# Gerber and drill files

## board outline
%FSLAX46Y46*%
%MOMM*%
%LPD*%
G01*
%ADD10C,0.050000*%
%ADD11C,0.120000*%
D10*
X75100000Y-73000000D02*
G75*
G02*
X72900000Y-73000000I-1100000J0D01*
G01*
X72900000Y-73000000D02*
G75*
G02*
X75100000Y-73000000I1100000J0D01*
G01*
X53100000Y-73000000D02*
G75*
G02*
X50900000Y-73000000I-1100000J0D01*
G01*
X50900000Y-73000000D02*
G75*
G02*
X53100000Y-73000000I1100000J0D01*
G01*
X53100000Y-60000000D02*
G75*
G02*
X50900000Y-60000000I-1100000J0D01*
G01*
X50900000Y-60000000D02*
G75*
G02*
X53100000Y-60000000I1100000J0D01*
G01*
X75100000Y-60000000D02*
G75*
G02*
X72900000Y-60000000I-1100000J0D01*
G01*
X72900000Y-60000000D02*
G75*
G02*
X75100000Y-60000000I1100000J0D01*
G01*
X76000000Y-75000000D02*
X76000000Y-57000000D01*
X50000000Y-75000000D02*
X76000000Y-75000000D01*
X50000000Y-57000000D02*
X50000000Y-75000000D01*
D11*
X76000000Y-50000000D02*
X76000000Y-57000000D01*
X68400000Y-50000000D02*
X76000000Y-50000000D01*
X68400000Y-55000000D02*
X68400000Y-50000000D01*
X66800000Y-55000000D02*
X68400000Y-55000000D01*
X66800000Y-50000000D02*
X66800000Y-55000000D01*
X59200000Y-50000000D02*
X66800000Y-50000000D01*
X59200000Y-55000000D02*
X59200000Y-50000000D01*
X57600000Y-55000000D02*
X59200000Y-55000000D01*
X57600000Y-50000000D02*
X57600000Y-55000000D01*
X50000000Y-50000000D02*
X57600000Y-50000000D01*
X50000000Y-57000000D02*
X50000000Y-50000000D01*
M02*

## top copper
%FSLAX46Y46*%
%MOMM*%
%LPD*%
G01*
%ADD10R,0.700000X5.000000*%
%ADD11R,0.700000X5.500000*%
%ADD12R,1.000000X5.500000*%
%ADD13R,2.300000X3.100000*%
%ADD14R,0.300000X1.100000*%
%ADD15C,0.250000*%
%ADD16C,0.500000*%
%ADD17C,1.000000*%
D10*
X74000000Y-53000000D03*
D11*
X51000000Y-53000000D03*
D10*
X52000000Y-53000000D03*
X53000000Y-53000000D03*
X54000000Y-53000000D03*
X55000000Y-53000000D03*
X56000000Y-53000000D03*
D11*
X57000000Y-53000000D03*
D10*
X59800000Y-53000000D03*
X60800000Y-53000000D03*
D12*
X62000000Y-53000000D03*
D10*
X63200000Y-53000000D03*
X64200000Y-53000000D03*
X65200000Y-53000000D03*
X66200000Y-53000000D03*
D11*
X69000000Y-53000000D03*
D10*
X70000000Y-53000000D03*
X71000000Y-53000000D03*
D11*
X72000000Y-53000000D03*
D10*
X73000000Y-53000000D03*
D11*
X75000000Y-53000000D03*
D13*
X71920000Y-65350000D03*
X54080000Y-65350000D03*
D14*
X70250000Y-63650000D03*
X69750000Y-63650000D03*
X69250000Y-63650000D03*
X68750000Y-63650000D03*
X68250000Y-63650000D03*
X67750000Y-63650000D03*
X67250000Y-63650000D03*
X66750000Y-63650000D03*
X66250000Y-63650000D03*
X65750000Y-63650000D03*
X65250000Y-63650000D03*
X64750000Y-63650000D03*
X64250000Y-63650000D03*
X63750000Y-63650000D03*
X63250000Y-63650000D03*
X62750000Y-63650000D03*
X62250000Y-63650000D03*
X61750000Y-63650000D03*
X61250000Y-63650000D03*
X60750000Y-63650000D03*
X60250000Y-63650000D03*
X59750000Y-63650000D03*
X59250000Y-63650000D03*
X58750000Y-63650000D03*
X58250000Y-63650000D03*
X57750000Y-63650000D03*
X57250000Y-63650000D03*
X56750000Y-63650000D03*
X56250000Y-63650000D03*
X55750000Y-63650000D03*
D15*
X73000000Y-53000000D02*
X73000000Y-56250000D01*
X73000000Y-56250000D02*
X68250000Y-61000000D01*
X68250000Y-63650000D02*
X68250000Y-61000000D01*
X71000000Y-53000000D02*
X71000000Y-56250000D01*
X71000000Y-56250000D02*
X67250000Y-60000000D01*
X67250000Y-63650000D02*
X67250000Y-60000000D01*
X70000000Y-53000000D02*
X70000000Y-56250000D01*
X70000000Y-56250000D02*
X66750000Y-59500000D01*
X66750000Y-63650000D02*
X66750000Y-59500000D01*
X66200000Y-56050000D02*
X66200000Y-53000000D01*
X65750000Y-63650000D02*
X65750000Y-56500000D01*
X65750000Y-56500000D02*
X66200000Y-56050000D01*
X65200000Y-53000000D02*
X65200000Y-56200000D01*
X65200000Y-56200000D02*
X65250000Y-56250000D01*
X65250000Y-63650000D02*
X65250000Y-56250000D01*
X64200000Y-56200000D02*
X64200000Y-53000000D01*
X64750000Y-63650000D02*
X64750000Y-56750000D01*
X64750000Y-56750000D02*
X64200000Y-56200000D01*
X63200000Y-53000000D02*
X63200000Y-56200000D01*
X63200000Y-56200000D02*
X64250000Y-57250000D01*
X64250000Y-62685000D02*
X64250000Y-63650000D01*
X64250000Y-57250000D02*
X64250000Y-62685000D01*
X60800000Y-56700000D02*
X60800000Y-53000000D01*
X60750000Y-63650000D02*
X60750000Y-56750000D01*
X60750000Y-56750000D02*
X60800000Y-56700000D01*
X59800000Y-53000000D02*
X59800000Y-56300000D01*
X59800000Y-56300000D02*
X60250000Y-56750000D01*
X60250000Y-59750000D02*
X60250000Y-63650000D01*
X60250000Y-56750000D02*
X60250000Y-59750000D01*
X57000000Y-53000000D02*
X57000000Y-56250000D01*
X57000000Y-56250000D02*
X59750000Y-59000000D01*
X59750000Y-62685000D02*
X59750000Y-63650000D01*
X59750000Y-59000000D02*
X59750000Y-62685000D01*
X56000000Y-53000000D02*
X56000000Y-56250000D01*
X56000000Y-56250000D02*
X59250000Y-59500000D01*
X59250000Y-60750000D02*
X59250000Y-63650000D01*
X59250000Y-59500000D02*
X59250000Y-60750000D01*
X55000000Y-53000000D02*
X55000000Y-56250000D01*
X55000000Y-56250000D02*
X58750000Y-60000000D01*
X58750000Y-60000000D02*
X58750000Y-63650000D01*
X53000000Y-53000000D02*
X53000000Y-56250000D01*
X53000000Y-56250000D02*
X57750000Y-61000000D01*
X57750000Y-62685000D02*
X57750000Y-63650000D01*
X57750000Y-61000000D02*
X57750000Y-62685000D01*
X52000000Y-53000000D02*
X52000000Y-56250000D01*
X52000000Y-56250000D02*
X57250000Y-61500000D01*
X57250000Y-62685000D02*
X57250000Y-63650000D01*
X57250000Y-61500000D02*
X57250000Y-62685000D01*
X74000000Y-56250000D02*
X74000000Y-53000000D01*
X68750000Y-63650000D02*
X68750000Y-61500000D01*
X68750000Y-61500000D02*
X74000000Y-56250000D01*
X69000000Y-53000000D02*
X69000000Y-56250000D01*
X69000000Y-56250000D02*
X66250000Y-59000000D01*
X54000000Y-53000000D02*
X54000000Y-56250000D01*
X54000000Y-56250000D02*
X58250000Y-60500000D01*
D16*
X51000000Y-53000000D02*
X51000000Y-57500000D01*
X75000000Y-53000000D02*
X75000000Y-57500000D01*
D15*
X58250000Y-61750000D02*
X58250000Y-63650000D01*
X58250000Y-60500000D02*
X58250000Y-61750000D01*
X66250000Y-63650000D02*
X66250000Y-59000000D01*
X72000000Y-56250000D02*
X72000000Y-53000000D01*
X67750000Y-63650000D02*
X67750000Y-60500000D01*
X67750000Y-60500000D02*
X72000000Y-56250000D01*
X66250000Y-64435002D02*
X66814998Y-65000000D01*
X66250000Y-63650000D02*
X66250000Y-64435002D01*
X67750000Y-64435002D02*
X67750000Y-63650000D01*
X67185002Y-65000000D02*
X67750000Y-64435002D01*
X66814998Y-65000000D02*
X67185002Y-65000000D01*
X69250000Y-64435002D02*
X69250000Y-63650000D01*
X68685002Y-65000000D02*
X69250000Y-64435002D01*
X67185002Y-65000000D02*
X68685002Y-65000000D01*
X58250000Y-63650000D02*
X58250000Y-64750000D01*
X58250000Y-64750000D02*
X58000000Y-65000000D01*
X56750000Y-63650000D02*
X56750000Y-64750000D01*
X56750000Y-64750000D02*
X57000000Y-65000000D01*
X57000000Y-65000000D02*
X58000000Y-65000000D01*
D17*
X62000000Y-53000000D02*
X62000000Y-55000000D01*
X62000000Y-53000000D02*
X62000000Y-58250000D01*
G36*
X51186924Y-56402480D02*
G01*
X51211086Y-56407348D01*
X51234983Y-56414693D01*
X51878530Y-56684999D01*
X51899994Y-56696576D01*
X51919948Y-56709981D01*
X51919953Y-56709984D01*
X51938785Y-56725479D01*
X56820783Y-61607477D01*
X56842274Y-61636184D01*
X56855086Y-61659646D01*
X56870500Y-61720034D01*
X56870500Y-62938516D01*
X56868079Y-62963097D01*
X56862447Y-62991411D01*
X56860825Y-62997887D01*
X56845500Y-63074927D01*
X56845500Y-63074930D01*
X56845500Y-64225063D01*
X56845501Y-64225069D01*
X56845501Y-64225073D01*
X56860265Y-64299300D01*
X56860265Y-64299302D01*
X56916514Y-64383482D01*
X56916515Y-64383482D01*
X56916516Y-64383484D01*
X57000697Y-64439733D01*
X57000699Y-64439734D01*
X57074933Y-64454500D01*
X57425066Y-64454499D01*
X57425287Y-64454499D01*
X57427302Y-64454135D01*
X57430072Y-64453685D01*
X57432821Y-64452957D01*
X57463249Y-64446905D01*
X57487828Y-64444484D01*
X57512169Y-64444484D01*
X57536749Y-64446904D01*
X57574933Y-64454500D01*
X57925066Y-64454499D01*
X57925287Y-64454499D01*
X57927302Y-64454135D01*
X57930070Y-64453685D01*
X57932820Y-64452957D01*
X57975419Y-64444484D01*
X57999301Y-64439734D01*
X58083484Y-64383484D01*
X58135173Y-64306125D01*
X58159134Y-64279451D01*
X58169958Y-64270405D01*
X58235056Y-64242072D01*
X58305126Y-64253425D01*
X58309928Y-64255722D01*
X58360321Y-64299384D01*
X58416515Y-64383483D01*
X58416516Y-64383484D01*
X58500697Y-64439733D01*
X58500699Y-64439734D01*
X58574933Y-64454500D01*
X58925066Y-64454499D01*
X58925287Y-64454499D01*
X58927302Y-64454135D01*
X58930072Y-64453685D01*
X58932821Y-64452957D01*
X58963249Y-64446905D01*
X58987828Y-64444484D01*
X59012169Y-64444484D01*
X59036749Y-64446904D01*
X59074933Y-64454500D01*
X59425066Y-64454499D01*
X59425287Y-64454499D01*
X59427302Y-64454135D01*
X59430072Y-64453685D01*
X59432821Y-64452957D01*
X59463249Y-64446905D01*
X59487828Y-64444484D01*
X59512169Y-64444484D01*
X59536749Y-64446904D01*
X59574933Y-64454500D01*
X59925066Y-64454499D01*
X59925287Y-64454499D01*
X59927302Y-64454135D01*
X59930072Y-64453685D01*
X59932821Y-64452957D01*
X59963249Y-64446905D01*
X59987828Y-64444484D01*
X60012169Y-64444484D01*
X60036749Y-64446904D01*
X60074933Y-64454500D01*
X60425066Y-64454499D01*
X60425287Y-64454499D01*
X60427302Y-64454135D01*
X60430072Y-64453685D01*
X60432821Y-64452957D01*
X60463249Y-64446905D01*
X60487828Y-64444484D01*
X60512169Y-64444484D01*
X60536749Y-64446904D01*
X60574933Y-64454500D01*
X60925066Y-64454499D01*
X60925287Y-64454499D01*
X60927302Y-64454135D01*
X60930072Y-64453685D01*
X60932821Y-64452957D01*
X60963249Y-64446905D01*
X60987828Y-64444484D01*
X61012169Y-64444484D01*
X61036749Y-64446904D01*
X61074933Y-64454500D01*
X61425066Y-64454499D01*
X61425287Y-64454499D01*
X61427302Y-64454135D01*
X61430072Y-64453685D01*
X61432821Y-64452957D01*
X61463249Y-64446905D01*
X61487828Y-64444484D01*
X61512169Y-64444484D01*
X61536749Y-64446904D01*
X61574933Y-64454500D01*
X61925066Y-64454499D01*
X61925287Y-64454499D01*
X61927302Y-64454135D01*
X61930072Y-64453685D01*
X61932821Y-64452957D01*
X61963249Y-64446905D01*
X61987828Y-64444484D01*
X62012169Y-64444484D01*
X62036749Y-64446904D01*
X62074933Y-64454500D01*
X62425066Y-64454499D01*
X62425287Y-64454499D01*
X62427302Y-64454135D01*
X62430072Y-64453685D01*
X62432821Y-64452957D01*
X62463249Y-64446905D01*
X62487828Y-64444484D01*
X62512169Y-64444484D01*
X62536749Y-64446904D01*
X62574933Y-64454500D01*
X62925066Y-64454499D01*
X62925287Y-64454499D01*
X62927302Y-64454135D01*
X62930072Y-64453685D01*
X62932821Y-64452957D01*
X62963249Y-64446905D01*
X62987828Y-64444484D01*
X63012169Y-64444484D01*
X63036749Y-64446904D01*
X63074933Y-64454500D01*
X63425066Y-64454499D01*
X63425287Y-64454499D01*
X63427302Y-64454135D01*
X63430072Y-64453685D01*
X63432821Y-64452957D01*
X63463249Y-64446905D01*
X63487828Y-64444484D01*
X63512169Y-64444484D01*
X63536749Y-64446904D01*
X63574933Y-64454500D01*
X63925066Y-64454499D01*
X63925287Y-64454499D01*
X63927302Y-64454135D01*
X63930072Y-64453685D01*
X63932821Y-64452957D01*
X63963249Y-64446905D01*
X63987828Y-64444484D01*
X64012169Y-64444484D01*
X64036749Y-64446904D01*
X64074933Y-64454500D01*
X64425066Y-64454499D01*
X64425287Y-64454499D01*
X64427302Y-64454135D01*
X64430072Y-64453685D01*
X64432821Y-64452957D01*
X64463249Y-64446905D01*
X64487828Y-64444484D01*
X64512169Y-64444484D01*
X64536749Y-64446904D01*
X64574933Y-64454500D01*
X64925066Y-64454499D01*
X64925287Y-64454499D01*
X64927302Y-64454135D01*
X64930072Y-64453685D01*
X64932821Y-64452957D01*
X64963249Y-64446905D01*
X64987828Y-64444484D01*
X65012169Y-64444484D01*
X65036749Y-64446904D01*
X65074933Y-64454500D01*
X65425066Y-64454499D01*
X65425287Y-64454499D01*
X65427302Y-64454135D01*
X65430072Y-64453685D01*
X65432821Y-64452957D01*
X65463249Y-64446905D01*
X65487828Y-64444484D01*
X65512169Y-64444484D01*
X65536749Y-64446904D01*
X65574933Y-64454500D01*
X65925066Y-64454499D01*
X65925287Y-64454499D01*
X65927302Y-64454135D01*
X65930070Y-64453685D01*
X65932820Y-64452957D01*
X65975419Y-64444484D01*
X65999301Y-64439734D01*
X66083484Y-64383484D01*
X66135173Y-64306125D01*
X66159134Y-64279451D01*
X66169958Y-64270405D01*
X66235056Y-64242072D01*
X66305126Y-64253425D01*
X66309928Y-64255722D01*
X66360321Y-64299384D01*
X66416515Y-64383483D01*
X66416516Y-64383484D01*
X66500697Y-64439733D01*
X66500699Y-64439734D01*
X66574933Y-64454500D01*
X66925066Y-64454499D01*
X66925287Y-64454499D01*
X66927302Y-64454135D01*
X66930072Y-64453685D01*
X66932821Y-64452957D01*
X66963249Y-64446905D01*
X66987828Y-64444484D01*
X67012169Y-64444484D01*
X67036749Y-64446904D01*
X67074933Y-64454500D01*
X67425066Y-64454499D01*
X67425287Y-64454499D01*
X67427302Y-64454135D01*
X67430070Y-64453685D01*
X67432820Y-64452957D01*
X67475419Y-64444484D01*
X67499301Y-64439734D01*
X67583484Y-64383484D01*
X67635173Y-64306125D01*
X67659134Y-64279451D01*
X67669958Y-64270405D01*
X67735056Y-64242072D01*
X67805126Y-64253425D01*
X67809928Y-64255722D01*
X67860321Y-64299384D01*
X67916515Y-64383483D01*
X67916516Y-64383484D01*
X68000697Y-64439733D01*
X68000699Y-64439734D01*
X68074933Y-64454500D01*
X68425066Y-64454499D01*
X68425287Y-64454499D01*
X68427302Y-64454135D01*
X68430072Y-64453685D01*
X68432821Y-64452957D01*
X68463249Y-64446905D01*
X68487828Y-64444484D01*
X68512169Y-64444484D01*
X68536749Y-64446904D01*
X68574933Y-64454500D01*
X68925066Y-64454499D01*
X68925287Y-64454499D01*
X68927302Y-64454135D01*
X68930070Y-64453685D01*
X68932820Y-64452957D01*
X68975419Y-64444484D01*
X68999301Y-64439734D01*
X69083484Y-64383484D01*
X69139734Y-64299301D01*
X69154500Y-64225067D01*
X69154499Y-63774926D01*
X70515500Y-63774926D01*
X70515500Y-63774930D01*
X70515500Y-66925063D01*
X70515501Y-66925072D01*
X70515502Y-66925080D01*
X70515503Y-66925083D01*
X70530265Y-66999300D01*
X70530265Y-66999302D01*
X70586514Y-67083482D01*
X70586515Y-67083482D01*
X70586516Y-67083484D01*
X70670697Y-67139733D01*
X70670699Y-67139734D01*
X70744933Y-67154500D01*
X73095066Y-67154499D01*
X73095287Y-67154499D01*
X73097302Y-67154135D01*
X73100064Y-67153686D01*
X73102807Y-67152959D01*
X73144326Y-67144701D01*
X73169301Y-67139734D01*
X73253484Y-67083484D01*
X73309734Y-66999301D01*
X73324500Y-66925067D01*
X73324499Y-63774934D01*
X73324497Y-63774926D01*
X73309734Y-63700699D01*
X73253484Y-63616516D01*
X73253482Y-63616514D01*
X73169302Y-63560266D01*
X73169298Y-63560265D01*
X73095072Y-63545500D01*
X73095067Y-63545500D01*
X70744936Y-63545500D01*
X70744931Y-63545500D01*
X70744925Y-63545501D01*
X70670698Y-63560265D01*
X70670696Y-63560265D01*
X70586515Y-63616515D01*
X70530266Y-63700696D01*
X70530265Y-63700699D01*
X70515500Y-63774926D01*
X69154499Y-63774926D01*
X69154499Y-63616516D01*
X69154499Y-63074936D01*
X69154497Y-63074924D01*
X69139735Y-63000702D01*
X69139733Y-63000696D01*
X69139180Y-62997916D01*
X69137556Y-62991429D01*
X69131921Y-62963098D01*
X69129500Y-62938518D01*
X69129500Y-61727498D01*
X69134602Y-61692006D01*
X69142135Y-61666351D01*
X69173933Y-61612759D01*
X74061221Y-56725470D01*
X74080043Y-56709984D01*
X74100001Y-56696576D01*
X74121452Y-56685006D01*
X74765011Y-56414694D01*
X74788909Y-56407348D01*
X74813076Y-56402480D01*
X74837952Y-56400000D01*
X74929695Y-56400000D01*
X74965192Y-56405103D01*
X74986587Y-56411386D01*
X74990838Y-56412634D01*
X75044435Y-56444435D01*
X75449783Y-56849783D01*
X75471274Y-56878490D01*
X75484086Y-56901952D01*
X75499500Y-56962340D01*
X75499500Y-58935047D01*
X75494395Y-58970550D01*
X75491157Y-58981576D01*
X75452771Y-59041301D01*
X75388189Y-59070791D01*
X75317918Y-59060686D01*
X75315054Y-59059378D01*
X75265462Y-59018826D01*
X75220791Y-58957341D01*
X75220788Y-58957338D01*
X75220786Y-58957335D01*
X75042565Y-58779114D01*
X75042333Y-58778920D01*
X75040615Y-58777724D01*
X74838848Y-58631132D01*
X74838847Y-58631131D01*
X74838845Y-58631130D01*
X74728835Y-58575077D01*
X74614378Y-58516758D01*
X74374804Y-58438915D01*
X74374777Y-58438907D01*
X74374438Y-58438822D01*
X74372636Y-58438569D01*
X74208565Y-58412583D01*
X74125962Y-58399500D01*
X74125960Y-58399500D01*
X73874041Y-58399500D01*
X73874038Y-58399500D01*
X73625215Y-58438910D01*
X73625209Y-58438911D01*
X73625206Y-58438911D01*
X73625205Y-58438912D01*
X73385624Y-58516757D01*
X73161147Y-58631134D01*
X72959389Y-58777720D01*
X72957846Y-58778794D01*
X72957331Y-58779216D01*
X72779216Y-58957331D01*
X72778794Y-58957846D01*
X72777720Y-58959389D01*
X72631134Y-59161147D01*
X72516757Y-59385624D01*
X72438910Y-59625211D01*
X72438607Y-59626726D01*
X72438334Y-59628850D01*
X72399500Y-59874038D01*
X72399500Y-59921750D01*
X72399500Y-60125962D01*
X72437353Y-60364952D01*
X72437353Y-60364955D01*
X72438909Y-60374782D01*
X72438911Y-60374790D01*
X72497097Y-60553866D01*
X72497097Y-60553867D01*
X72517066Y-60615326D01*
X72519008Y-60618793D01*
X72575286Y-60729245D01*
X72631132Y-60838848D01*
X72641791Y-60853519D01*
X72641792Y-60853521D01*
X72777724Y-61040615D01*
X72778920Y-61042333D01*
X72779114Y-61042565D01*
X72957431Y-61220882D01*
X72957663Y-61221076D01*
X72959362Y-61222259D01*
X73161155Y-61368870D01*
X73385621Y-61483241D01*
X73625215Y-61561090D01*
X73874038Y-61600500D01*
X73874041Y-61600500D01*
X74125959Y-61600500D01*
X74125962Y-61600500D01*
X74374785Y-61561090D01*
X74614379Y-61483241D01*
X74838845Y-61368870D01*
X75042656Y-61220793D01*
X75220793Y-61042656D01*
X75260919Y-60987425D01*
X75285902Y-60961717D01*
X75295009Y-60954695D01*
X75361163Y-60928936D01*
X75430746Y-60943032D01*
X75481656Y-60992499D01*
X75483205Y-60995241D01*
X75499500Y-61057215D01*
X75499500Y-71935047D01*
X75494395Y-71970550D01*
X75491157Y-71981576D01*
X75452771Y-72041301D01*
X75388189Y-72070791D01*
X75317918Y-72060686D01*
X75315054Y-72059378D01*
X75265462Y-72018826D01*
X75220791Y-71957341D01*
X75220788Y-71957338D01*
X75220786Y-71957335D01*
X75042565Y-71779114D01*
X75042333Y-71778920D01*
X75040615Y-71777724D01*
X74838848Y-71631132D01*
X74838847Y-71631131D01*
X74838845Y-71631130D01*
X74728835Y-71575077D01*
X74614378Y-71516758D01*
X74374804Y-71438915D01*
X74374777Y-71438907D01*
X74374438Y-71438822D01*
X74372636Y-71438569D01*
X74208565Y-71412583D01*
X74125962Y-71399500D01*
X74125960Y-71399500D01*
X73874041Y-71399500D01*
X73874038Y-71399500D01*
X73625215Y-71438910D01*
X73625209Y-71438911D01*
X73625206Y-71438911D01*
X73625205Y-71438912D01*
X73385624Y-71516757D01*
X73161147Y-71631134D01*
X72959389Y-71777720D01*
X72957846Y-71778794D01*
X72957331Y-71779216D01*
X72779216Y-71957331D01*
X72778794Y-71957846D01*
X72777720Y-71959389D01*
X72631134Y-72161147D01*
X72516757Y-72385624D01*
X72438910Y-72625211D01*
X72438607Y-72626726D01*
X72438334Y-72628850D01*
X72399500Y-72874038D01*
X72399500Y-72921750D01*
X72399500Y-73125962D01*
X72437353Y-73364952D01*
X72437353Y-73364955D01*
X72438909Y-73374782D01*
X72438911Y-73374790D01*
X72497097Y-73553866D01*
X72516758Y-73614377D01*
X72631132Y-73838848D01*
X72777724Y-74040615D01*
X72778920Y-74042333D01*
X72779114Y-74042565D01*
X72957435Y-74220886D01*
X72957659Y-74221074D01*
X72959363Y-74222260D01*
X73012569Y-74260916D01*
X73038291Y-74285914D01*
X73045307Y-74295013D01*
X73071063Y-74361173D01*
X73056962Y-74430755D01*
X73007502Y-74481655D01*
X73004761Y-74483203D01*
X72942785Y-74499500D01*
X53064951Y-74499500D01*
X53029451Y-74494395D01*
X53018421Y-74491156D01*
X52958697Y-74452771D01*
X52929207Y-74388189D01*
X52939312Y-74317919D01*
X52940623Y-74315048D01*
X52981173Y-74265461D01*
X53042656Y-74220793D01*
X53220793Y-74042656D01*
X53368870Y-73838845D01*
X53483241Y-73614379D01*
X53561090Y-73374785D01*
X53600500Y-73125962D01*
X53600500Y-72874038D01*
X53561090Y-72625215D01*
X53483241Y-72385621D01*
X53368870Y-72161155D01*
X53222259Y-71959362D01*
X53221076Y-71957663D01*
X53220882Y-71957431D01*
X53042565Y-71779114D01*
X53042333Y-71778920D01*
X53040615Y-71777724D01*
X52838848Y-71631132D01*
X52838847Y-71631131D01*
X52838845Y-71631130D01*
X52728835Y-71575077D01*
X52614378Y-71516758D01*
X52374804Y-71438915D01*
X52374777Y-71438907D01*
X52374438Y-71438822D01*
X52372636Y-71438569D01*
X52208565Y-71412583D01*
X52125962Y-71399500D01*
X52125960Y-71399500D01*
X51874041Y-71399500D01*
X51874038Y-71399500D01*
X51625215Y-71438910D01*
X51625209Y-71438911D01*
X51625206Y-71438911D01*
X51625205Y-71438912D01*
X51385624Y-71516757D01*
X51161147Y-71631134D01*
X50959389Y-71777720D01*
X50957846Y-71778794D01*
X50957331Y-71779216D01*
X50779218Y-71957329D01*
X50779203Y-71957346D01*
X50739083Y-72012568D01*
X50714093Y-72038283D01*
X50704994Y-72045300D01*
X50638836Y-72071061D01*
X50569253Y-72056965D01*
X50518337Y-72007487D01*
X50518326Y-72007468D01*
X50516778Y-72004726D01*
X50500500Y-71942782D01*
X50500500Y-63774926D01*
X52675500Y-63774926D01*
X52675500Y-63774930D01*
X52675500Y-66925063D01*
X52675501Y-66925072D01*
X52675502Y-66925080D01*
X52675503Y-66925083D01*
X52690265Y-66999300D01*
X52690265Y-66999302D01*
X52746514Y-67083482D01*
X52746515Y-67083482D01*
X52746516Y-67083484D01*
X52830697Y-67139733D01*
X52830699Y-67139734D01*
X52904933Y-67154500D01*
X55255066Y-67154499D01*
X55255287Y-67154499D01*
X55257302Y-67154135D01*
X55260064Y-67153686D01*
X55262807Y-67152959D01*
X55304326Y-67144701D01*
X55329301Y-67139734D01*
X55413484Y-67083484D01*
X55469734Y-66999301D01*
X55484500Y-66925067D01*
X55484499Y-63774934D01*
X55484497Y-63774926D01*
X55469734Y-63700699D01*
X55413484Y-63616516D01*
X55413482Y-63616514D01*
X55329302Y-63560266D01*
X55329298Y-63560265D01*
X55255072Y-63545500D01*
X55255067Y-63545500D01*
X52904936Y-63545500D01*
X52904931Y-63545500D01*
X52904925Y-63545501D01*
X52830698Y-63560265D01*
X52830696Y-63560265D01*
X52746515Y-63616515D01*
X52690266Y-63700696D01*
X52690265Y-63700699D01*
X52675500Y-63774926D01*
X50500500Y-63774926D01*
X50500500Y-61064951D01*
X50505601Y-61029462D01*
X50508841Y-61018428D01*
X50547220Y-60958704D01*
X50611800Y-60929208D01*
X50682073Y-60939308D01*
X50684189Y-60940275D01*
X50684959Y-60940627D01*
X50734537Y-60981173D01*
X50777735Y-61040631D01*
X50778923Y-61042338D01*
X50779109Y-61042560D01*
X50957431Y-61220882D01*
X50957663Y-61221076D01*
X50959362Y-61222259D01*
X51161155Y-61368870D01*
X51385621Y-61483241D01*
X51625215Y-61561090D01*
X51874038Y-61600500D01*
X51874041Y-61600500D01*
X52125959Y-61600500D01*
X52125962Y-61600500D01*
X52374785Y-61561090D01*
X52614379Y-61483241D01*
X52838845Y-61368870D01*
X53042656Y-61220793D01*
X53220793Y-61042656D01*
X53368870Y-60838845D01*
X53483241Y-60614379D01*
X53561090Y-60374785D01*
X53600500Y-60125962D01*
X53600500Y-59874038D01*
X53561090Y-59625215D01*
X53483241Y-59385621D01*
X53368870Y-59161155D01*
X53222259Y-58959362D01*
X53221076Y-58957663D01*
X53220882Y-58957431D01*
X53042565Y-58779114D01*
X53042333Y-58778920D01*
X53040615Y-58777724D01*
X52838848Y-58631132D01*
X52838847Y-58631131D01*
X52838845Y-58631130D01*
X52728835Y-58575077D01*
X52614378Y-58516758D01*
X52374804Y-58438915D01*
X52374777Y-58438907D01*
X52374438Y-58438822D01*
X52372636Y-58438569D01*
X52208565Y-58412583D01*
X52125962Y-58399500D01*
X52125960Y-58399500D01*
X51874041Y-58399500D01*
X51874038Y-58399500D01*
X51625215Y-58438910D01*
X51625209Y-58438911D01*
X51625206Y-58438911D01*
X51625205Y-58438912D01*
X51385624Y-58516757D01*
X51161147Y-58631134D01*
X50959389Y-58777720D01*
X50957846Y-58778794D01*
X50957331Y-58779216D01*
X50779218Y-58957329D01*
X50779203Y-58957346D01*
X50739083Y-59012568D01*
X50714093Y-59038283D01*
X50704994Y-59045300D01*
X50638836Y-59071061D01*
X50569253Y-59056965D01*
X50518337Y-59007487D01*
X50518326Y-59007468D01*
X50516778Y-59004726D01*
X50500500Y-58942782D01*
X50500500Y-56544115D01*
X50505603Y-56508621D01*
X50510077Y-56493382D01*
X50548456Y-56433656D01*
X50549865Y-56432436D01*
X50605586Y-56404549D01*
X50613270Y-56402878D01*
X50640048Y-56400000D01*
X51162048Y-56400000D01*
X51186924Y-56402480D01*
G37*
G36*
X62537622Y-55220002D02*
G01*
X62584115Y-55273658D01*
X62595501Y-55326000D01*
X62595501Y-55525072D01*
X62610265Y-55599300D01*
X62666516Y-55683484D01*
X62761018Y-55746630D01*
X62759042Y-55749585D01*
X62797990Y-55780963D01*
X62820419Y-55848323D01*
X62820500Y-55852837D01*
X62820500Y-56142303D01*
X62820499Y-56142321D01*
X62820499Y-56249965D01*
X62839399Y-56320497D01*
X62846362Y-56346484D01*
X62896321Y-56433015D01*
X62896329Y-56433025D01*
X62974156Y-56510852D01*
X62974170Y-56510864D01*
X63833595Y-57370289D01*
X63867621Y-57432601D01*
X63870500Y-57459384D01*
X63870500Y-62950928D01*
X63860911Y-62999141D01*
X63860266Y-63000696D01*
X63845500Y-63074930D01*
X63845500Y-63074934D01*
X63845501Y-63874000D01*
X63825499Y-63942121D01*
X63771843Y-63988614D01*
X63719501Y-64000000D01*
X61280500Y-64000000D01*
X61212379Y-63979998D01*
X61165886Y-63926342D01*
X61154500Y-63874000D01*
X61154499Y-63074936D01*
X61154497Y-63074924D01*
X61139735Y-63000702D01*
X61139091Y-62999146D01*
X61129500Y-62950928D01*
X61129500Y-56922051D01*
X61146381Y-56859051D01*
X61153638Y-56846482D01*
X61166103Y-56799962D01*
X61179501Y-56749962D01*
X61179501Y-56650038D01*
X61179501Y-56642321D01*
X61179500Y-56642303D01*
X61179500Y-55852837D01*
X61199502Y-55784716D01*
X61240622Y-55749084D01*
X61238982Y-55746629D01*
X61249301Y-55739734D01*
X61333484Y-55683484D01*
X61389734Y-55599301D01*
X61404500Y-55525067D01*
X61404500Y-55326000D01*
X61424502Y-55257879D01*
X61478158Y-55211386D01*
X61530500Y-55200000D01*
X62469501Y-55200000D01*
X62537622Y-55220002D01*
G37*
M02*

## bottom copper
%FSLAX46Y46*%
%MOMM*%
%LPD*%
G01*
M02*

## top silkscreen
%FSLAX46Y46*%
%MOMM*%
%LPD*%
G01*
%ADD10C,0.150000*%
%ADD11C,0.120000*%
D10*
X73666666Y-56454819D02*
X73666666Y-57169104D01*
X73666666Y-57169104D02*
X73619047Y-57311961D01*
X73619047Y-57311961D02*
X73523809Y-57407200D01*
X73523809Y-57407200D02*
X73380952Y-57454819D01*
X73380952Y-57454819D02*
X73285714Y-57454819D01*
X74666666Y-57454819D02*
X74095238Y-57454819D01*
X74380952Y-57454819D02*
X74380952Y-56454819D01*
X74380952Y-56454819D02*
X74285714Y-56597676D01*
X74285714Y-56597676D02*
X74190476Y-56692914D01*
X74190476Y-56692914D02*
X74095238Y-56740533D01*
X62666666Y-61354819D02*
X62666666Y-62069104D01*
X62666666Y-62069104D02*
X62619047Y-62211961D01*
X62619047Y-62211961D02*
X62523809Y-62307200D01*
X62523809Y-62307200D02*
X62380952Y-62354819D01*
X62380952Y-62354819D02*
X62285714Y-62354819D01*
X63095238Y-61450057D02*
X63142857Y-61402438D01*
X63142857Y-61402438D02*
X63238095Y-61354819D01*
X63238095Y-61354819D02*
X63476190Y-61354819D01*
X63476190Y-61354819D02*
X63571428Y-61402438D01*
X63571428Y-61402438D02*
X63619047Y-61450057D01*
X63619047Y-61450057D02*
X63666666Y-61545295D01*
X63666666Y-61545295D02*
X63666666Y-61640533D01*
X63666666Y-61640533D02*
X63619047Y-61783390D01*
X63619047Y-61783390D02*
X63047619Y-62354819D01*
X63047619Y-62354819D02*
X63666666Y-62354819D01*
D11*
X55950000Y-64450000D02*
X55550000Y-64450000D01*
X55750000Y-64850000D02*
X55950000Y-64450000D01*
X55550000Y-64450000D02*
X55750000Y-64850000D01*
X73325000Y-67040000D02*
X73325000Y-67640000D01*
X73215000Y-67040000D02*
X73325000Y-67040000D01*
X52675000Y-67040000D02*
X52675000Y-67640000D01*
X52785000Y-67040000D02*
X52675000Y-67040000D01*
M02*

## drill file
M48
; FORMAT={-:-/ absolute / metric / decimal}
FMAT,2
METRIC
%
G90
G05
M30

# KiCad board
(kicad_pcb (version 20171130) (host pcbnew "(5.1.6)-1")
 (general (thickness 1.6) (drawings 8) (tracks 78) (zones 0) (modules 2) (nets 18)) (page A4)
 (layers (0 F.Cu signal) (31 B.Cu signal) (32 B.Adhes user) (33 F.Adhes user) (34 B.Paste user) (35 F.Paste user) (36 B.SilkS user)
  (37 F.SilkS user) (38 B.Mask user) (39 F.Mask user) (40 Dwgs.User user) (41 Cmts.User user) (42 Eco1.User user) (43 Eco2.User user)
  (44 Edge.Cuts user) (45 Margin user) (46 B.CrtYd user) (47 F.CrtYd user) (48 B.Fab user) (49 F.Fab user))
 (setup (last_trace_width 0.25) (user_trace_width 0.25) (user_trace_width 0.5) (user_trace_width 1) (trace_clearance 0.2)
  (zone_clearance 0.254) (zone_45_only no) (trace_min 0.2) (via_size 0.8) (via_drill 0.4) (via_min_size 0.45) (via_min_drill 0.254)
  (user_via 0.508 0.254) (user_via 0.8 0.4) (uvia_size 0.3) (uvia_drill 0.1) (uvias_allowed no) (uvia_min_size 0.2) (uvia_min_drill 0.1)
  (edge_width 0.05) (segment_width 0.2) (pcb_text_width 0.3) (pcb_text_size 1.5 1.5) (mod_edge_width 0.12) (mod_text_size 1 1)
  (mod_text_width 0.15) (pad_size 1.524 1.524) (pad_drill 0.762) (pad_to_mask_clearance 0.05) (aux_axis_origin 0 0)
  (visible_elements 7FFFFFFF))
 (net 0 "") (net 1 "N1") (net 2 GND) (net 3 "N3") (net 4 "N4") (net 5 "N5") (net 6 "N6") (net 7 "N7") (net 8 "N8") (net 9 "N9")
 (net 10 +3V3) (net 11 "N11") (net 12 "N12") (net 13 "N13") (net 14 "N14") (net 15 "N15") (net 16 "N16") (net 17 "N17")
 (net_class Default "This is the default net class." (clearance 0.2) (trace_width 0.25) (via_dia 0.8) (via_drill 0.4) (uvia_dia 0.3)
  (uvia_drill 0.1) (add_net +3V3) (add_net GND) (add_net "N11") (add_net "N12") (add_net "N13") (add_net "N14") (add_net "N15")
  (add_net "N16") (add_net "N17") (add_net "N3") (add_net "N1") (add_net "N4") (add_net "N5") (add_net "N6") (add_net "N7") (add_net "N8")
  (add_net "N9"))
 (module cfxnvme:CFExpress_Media (layer F.Cu) (at 49 48)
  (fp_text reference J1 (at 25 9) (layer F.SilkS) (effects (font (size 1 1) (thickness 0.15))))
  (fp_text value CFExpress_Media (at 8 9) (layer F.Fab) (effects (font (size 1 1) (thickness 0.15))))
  (fp_line (start 27 2) (end 27 9) (layer Edge.Cuts) (width 0.12))
  (fp_line (start 19.4 2) (end 27 2) (layer Edge.Cuts) (width 0.12))
  (fp_line (start 19.4 7) (end 19.4 2) (layer Edge.Cuts) (width 0.12))
  (fp_line (start 17.8 7) (end 19.4 7) (layer Edge.Cuts) (width 0.12))
  (fp_line (start 17.8 2) (end 17.8 7) (layer Edge.Cuts) (width 0.12))
  (fp_line (start 10.2 2) (end 17.8 2) (layer Edge.Cuts) (width 0.12))
  (fp_line (start 10.2 7) (end 10.2 2) (layer Edge.Cuts) (width 0.12))
  (fp_line (start 8.6 7) (end 10.2 7) (layer Edge.Cuts) (width 0.12))
  (fp_line (start 8.6 2) (end 8.6 7) (layer Edge.Cuts) (width 0.12))
  (fp_line (start 1 2) (end 8.6 2) (layer Edge.Cuts) (width 0.12))
  (fp_line (start 1 9) (end 1 2) (layer Edge.Cuts) (width 0.12))
  (pad 20 connect rect (at 25 5) (size 0.7 5) (layers F.Cu F.Mask) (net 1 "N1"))
  (pad 1 connect rect (at 2 5) (size 0.7 5.5) (layers F.Cu F.Mask) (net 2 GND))
  (pad 2 connect rect (at 3 5) (size 0.7 5) (layers F.Cu F.Mask) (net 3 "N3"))
  (pad 3 connect rect (at 4 5) (size 0.7 5) (layers F.Cu F.Mask) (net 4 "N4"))
  (pad 4 connect rect (at 5 5) (size 0.7 5) (layers F.Cu F.Mask) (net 2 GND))
  (pad 5 connect rect (at 6 5) (size 0.7 5) (layers F.Cu F.Mask) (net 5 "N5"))
  (pad 6 connect rect (at 7 5) (size 0.7 5) (layers F.Cu F.Mask) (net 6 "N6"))
  (pad 7 connect rect (at 8 5) (size 0.7 5.5) (layers F.Cu F.Mask) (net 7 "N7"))
  (pad 8 connect rect (at 10.8 5) (size 0.7 5) (layers F.Cu F.Mask) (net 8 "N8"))
  (pad 9 connect rect (at 11.8 5) (size 0.7 5) (layers F.Cu F.Mask) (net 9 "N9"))
  (pad 10 connect rect (at 13 5) (size 1 5.5) (layers F.Cu F.Mask) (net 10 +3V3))
  (pad 11 connect rect (at 14.2 5) (size 0.7 5) (layers F.Cu F.Mask) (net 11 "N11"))
  (pad 12 connect rect (at 15.2 5) (size 0.7 5) (layers F.Cu F.Mask) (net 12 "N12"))
  (pad 13 connect rect (at 16.2 5) (size 0.7 5) (layers F.Cu F.Mask) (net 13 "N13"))
  (pad 14 connect rect (at 17.2 5) (size 0.7 5) (layers F.Cu F.Mask) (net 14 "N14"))
  (pad 15 connect rect (at 20 5) (size 0.7 5.5) (layers F.Cu F.Mask) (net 2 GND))
  (pad 16 connect rect (at 21 5) (size 0.7 5) (layers F.Cu F.Mask) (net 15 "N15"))
  (pad 17 connect rect (at 22 5) (size 0.7 5) (layers F.Cu F.Mask) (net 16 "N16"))
  (pad 18 connect rect (at 23 5) (size 0.7 5.5) (layers F.Cu F.Mask) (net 2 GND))
  (pad 19 connect rect (at 24 5) (size 0.7 5) (layers F.Cu F.Mask) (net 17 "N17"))
  (pad 21 connect rect (at 26 5) (size 0.7 5.5) (layers F.Cu F.Mask) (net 2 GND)))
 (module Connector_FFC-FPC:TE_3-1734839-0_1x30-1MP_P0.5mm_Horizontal (layer F.Cu) (at 63 65)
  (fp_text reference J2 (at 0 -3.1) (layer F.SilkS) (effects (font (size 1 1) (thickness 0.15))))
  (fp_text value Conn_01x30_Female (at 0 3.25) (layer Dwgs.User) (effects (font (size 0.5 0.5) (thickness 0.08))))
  (fp_line (start -7.05 -0.55) (end -7.45 -0.55) (layer F.SilkS) (width 0.12))
  (fp_line (start -7.25 -0.15) (end -7.05 -0.55) (layer F.SilkS) (width 0.12))
  (fp_line (start -7.45 -0.55) (end -7.25 -0.15) (layer F.SilkS) (width 0.12))
  (fp_line (start 10.325 2.04) (end 10.325 2.64) (layer F.SilkS) (width 0.12))
  (fp_line (start 10.215 2.04) (end 10.325 2.04) (layer F.SilkS) (width 0.12))
  (fp_line (start -10.325 2.04) (end -10.325 2.64) (layer F.SilkS) (width 0.12))
  (fp_line (start -10.215 2.04) (end -10.325 2.04) (layer F.SilkS) (width 0.12))
  (pad MP smd rect (at 8.92 0.35) (size 2.3 3.1) (layers F.Cu F.Paste F.Mask))
  (pad MP smd rect (at -8.92 0.35) (size 2.3 3.1) (layers F.Cu F.Paste F.Mask))
  (pad 30 smd rect (at 7.25 -1.35) (size 0.3 1.1) (layers F.Cu F.Paste F.Mask) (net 2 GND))
  (pad 29 smd rect (at 6.75 -1.35) (size 0.3 1.1) (layers F.Cu F.Paste F.Mask) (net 2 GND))
  (pad 28 smd rect (at 6.25 -1.35) (size 0.3 1.1) (layers F.Cu F.Paste F.Mask) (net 2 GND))
  (pad 27 smd rect (at 5.75 -1.35) (size 0.3 1.1) (layers F.Cu F.Paste F.Mask) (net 1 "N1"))
  (pad 26 smd rect (at 5.25 -1.35) (size 0.3 1.1) (layers F.Cu F.Paste F.Mask) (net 17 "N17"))
  (pad 25 smd rect (at 4.75 -1.35) (size 0.3 1.1) (layers F.Cu F.Paste F.Mask) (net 2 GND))
  (pad 24 smd rect (at 4.25 -1.35) (size 0.3 1.1) (layers F.Cu F.Paste F.Mask) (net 16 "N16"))
  (pad 23 smd rect (at 3.75 -1.35) (size 0.3 1.1) (layers F.Cu F.Paste F.Mask) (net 15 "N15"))
  (pad 22 smd rect (at 3.25 -1.35) (size 0.3 1.1) (layers F.Cu F.Paste F.Mask) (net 2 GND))
  (pad 21 smd rect (at 2.75 -1.35) (size 0.3 1.1) (layers F.Cu F.Paste F.Mask) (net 14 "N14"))
  (pad 20 smd rect (at 2.25 -1.35) (size 0.3 1.1) (layers F.Cu F.Paste F.Mask) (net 13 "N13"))
  (pad 19 smd rect (at 1.75 -1.35) (size 0.3 1.1) (layers F.Cu F.Paste F.Mask) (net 12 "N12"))
  (pad 18 smd rect (at 1.25 -1.35) (size 0.3 1.1) (layers F.Cu F.Paste F.Mask) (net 11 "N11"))
  (pad 17 smd rect (at 0.75 -1.35) (size 0.3 1.1) (layers F.Cu F.Paste F.Mask) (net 10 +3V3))
  (pad 16 smd rect (at 0.25 -1.35) (size 0.3 1.1) (layers F.Cu F.Paste F.Mask) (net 10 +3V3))
  (pad 15 smd rect (at -0.25 -1.35) (size 0.3 1.1) (layers F.Cu F.Paste F.Mask) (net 10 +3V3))
  (pad 14 smd rect (at -0.75 -1.35) (size 0.3 1.1) (layers F.Cu F.Paste F.Mask) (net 10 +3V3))
  (pad 13 smd rect (at -1.25 -1.35) (size 0.3 1.1) (layers F.Cu F.Paste F.Mask) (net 10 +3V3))
  (pad 12 smd rect (at -1.75 -1.35) (size 0.3 1.1) (layers F.Cu F.Paste F.Mask) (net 10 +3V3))
  (pad 11 smd rect (at -2.25 -1.35) (size 0.3 1.1) (layers F.Cu F.Paste F.Mask) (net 9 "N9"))
  (pad 10 smd rect (at -2.75 -1.35) (size 0.3 1.1) (layers F.Cu F.Paste F.Mask) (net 8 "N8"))
  (pad 9 smd rect (at -3.25 -1.35) (size 0.3 1.1) (layers F.Cu F.Paste F.Mask) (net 7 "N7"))
  (pad 8 smd rect (at -3.75 -1.35) (size 0.3 1.1) (layers F.Cu F.Paste F.Mask) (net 6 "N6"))
  (pad 7 smd rect (at -4.25 -1.35) (size 0.3 1.1) (layers F.Cu F.Paste F.Mask) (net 5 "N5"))
  (pad 6 smd rect (at -4.75 -1.35) (size 0.3 1.1) (layers F.Cu F.Paste F.Mask) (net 2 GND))
  (pad 5 smd rect (at -5.25 -1.35) (size 0.3 1.1) (layers F.Cu F.Paste F.Mask) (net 4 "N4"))
  (pad 4 smd rect (at -5.75 -1.35) (size 0.3 1.1) (layers F.Cu F.Paste F.Mask) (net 3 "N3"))
  (pad 3 smd rect (at -6.25 -1.35) (size 0.3 1.1) (layers F.Cu F.Paste F.Mask) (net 2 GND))
  (pad 2 smd rect (at -6.75 -1.35) (size 0.3 1.1) (layers F.Cu F.Paste F.Mask) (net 2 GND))
  (pad 1 smd rect (at -7.25 -1.35) (size 0.3 1.1) (layers F.Cu F.Paste F.Mask) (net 2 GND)))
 (gr_circle (center 74 73) (end 75.1 73) (layer Edge.Cuts) (width 0.05))
 (gr_circle (center 52 73) (end 53.1 73) (layer Edge.Cuts) (width 0.05))
 (gr_circle (center 52 60) (end 53.1 60) (layer Edge.Cuts) (width 0.05))
 (gr_circle (center 74 60) (end 75.1 60) (layer Edge.Cuts) (width 0.05))
 (gr_line (start 76 75) (end 76 57) (angle 90) (layer Edge.Cuts) (width 0.05))
 (gr_line (start 50 75) (end 76 75) (angle 90) (layer Edge.Cuts) (width 0.05))
 (gr_line (start 50 57) (end 50 75) (angle 90) (layer Edge.Cuts) (width 0.05))
 (segment (start 73 53) (end 73 56.25) (width 0.25) (layer F.Cu) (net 17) (status 400000))
 (segment (start 73 56.25) (end 68.25 61) (width 0.25) (layer F.Cu) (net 17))
 (segment (start 68.25 63.65) (end 68.25 61) (width 0.25) (layer F.Cu) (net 17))
 (segment (start 71 53) (end 71 56.25) (width 0.25) (layer F.Cu) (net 16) (status 400000))
 (segment (start 71 56.25) (end 67.25 60) (width 0.25) (layer F.Cu) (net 16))
 (segment (start 67.25 63.65) (end 67.25 60) (width 0.25) (layer F.Cu) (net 16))
 (segment (start 70 53) (end 70 56.25) (width 0.25) (layer F.Cu) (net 15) (status 400000))
 (segment (start 70 56.25) (end 66.75 59.5) (width 0.25) (layer F.Cu) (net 15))
 (segment (start 66.75 63.65) (end 66.75 59.5) (width 0.25) (layer F.Cu) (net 15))
 (segment (start 66.2 56.05) (end 66.2 53) (width 0.25) (layer F.Cu) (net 14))
 (segment (start 65.75 63.65) (end 65.75 56.5) (width 0.25) (layer F.Cu) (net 14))
 (segment (start 65.75 56.5) (end 66.2 56.05) (width 0.25) (layer F.Cu) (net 14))
 (segment (start 65.2 53) (end 65.2 56.2) (width 0.25) (layer F.Cu) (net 13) (status 400000))
 (segment (start 65.2 56.2) (end 65.25 56.25) (width 0.25) (layer F.Cu) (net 13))
 (segment (start 65.25 63.65) (end 65.25 56.25) (width 0.25) (layer F.Cu) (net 13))
 (segment (start 64.2 56.2) (end 64.2 53) (width 0.25) (layer F.Cu) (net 12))
 (segment (start 64.75 63.65) (end 64.75 56.75) (width 0.25) (layer F.Cu) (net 12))
 (segment (start 64.75 56.75) (end 64.2 56.2) (width 0.25) (layer F.Cu) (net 12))
 (segment (start 63.2 53) (end 63.2 56.2) (width 0.25) (layer F.Cu) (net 11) (status 400000))
 (segment (start 63.2 56.2) (end 64.25 57.25) (width 0.25) (layer F.Cu) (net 11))
 (segment (start 64.25 62.685) (end 64.25 63.65) (width 0.25) (layer F.Cu) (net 11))
 (segment (start 64.25 57.25) (end 64.25 62.685) (width 0.25) (layer F.Cu) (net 11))
 (segment (start 60.8 56.7) (end 60.8 53) (width 0.25) (layer F.Cu) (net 9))
 (segment (start 60.75 63.65) (end 60.75 56.75) (width 0.25) (layer F.Cu) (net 9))
 (segment (start 60.75 56.75) (end 60.8 56.7) (width 0.25) (layer F.Cu) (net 9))
 (segment (start 59.8 53) (end 59.8 56.3) (width 0.25) (layer F.Cu) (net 8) (status 400000))
 (segment (start 59.8 56.3) (end 60.25 56.75) (width 0.25) (layer F.Cu) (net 8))
 (segment (start 60.25 59.75) (end 60.25 63.65) (width 0.25) (layer F.Cu) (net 8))
 (segment (start 60.25 56.75) (end 60.25 59.75) (width 0.25) (layer F.Cu) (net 8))
 (segment (start 57 53) (end 57 56.25) (width 0.25) (layer F.Cu) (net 7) (status 400000))
 (segment (start 57 56.25) (end 59.75 59) (width 0.25) (layer F.Cu) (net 7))
 (segment (start 59.75 62.685) (end 59.75 63.65) (width 0.25) (layer F.Cu) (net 7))
 (segment (start 59.75 59) (end 59.75 62.685) (width 0.25) (layer F.Cu) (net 7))
 (segment (start 56 53) (end 56 56.25) (width 0.25) (layer F.Cu) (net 6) (status 400000))
 (segment (start 56 56.25) (end 59.25 59.5) (width 0.25) (layer F.Cu) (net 6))
 (segment (start 59.25 60.75) (end 59.25 63.65) (width 0.25) (layer F.Cu) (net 6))
 (segment (start 59.25 59.5) (end 59.25 60.75) (width 0.25) (layer F.Cu) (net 6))
 (segment (start 55 53) (end 55 56.25) (width 0.25) (layer F.Cu) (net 5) (status 400000))
 (segment (start 55 56.25) (end 58.75 60) (width 0.25) (layer F.Cu) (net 5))
 (segment (start 58.75 60) (end 58.75 63.65) (width 0.25) (layer F.Cu) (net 5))
 (segment (start 53 53) (end 53 56.25) (width 0.25) (layer F.Cu) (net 4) (status 400000))
 (segment (start 53 56.25) (end 57.75 61) (width 0.25) (layer F.Cu) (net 4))
 (segment (start 57.75 62.685) (end 57.75 63.65) (width 0.25) (layer F.Cu) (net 4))
 (segment (start 57.75 61) (end 57.75 62.685) (width 0.25) (layer F.Cu) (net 4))
 (segment (start 52 53) (end 52 56.25) (width 0.25) (layer F.Cu) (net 3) (status 400000))
 (segment (start 52 56.25) (end 57.25 61.5) (width 0.25) (layer F.Cu) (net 3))
 (segment (start 57.25 62.685) (end 57.25 63.65) (width 0.25) (layer F.Cu) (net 3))
 (segment (start 57.25 61.5) (end 57.25 62.685) (width 0.25) (layer F.Cu) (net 3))
 (segment (start 74 56.25) (end 74 53) (width 0.25) (layer F.Cu) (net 1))
 (segment (start 68.75 63.65) (end 68.75 61.5) (width 0.25) (layer F.Cu) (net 1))
 (segment (start 68.75 61.5) (end 74 56.25) (width 0.25) (layer F.Cu) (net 1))
 (segment (start 69 53) (end 69 56.25) (width 0.25) (layer F.Cu) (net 2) (status 400000))
 (segment (start 69 56.25) (end 66.25 59) (width 0.25) (layer F.Cu) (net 2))
 (segment (start 54 53) (end 54 56.25) (width 0.25) (layer F.Cu) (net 2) (status 400000))
 (segment (start 54 56.25) (end 58.25 60.5) (width 0.25) (layer F.Cu) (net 2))
 (segment (start 51 53) (end 51 57.5) (width 0.5) (layer F.Cu) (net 2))
 (segment (start 75 53) (end 75 57.5) (width 0.5) (layer F.Cu) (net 2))
 (segment (start 58.25 61.75) (end 58.25 63.65) (width 0.25) (layer F.Cu) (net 2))
 (segment (start 58.25 60.5) (end 58.25 61.75) (width 0.25) (layer F.Cu) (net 2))
 (segment (start 66.25 63.65) (end 66.25 59) (width 0.25) (layer F.Cu) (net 2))
 (segment (start 72 56.25) (end 72 53) (width 0.25) (layer F.Cu) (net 2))
 (segment (start 67.75 63.65) (end 67.75 60.5) (width 0.25) (layer F.Cu) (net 2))
 (segment (start 67.75 60.5) (end 72 56.25) (width 0.25) (layer F.Cu) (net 2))
 (segment (start 66.25 64.435002) (end 66.814998 65) (width 0.25) (layer F.Cu) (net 2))
 (segment (start 66.25 63.65) (end 66.25 64.435002) (width 0.25) (layer F.Cu) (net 2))
 (segment (start 67.75 64.435002) (end 67.75 63.65) (width 0.25) (layer F.Cu) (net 2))
 (segment (start 67.185002 65) (end 67.75 64.435002) (width 0.25) (layer F.Cu) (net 2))
 (segment (start 66.814998 65) (end 67.185002 65) (width 0.25) (layer F.Cu) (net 2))
 (segment (start 69.25 64.435002) (end 69.25 63.65) (width 0.25) (layer F.Cu) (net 2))
 (segment (start 68.685002 65) (end 69.25 64.435002) (width 0.25) (layer F.Cu) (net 2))
 (segment (start 67.185002 65) (end 68.685002 65) (width 0.25) (layer F.Cu) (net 2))
 (segment (start 58.25 63.65) (end 58.25 64.75) (width 0.25) (layer F.Cu) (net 2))
 (segment (start 58.25 64.75) (end 58 65) (width 0.25) (layer F.Cu) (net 2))
 (segment (start 56.75 63.65) (end 56.75 64.75) (width 0.25) (layer F.Cu) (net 2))
 (segment (start 56.75 64.75) (end 57 65) (width 0.25) (layer F.Cu) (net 2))
 (segment (start 57 65) (end 58 65) (width 0.25) (layer F.Cu) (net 2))
 (segment (start 62 53) (end 62 55) (width 1) (layer F.Cu) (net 10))
 (segment (start 62 53) (end 62 58.25) (width 1) (layer F.Cu) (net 10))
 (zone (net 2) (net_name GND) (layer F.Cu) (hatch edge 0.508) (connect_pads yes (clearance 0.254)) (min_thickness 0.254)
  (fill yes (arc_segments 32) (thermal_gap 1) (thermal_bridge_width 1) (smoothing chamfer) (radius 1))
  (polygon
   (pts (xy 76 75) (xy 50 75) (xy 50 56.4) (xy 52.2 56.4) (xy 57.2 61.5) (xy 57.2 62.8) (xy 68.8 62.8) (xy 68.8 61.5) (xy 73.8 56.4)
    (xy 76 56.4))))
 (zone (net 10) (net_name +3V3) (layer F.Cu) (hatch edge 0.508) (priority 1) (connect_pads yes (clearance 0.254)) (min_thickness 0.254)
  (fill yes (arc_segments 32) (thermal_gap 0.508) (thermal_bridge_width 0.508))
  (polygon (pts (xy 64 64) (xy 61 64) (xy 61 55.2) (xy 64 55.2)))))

